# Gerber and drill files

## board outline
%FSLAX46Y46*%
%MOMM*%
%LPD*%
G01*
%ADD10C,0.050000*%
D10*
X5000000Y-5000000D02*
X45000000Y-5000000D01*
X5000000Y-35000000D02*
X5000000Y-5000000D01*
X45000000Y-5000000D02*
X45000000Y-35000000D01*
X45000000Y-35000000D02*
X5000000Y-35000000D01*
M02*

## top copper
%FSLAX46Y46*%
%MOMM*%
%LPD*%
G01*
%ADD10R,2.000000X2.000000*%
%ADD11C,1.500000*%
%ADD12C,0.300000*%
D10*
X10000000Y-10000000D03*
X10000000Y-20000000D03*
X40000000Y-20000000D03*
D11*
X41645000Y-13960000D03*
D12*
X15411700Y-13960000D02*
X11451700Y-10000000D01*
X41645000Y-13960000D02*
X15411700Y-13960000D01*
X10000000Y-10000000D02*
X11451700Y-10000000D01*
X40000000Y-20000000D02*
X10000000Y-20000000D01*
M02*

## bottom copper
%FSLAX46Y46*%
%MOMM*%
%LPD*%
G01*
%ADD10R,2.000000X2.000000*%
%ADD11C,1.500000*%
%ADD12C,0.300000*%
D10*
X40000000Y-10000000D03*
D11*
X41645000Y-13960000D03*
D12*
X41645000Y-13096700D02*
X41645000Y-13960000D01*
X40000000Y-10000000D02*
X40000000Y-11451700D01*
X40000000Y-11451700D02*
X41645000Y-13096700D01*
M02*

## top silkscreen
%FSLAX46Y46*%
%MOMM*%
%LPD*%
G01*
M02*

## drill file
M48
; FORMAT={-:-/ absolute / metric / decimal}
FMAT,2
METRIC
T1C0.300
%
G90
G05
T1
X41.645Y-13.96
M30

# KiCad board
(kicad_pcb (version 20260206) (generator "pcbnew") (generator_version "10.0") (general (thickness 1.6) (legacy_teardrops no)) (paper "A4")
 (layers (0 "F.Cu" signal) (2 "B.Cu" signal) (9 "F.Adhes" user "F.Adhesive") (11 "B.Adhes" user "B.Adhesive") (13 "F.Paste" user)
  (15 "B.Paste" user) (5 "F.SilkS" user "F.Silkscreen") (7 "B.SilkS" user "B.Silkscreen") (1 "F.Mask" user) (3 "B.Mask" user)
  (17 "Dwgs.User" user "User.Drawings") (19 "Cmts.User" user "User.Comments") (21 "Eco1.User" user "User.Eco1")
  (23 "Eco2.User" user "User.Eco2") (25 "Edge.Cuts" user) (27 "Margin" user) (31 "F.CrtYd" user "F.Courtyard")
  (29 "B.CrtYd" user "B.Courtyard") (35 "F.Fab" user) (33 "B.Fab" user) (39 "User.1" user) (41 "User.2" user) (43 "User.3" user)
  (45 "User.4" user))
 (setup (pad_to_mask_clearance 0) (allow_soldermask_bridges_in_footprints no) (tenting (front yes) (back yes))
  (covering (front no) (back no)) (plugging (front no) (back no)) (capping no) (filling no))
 (gr_line (start 5 5) (end 45 5) (stroke (width 0.05) (type default)) (layer "Edge.Cuts"))
 (gr_line (start 5 35) (end 5 5) (stroke (width 0.05) (type default)) (layer "Edge.Cuts"))
 (gr_line (start 45 5) (end 45 35) (stroke (width 0.05) (type default)) (layer "Edge.Cuts"))
 (gr_line (start 45 35) (end 5 35) (stroke (width 0.05) (type default)) (layer "Edge.Cuts"))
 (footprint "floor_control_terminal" (layer "F.Cu") (at 10 10)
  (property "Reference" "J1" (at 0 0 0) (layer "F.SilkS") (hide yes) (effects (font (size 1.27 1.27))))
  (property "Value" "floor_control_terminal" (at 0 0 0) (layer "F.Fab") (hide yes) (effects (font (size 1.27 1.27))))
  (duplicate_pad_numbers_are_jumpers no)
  (pad "1" smd rect (at 0 0) (size 2 2) (layers "F.Cu" "F.Paste" "F.Mask") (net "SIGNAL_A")))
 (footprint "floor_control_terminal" (layer "B.Cu") (at 40 10)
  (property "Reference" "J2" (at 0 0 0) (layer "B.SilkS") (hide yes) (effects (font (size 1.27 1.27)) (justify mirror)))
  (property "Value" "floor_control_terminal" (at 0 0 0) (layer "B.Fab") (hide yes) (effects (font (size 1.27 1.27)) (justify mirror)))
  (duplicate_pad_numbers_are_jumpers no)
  (pad "1" smd rect (at 0 0) (size 2 2) (layers "B.Cu" "B.Paste" "B.Mask") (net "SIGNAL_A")))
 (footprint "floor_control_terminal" (layer "F.Cu") (at 10 20)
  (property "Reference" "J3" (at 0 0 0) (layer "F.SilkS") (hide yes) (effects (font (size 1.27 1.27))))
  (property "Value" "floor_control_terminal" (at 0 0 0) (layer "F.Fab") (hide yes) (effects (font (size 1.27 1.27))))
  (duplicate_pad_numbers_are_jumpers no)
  (pad "1" smd rect (at 0 0) (size 2 2) (layers "F.Cu" "F.Paste" "F.Mask") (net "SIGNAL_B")))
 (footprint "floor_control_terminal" (layer "F.Cu") (at 40 20)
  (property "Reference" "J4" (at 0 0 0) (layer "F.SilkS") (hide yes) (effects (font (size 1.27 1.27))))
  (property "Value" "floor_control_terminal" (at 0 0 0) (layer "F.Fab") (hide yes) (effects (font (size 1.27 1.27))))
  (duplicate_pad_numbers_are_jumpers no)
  (pad "1" smd rect (at 0 0) (size 2 2) (layers "F.Cu" "F.Paste" "F.Mask") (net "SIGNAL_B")))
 (segment (start 15.4117 13.96) (end 11.4517 10) (width 0.3) (layer "F.Cu") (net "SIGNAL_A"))
 (segment (start 41.645 13.96) (end 15.4117 13.96) (width 0.3) (layer "F.Cu") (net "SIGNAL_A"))
 (segment (start 10 10) (end 11.4517 10) (width 0.3) (layer "F.Cu") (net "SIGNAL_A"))
 (via (at 41.645 13.96) (size 1.5) (drill 0.3) (layers "F.Cu" "B.Cu") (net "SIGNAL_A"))
 (segment (start 41.645 13.0967) (end 41.645 13.96) (width 0.3) (layer "B.Cu") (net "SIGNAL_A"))
 (segment (start 40 10) (end 40 11.4517) (width 0.3) (layer "B.Cu") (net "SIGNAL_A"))
 (segment (start 40 11.4517) (end 41.645 13.0967) (width 0.3) (layer "B.Cu") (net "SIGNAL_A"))
 (segment (start 40 20) (end 10 20) (width 0.3) (layer "F.Cu") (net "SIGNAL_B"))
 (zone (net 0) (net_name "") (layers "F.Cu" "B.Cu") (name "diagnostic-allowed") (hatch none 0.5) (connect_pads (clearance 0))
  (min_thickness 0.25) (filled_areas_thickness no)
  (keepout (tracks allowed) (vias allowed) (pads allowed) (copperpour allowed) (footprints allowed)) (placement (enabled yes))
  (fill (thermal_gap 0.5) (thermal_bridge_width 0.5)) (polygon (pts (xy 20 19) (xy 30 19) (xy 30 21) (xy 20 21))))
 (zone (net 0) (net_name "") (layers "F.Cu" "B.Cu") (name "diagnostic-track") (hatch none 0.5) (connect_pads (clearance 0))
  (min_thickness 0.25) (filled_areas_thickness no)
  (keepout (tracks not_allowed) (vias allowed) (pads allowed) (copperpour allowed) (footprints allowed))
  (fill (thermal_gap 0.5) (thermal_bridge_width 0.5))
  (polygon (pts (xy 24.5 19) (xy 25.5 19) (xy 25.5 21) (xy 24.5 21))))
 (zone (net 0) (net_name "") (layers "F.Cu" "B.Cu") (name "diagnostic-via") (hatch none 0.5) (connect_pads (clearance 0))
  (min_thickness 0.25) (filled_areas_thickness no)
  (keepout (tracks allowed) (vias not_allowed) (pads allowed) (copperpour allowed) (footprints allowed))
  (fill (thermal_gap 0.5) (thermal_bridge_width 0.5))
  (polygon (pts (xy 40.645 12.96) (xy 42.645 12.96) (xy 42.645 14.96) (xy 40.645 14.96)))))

